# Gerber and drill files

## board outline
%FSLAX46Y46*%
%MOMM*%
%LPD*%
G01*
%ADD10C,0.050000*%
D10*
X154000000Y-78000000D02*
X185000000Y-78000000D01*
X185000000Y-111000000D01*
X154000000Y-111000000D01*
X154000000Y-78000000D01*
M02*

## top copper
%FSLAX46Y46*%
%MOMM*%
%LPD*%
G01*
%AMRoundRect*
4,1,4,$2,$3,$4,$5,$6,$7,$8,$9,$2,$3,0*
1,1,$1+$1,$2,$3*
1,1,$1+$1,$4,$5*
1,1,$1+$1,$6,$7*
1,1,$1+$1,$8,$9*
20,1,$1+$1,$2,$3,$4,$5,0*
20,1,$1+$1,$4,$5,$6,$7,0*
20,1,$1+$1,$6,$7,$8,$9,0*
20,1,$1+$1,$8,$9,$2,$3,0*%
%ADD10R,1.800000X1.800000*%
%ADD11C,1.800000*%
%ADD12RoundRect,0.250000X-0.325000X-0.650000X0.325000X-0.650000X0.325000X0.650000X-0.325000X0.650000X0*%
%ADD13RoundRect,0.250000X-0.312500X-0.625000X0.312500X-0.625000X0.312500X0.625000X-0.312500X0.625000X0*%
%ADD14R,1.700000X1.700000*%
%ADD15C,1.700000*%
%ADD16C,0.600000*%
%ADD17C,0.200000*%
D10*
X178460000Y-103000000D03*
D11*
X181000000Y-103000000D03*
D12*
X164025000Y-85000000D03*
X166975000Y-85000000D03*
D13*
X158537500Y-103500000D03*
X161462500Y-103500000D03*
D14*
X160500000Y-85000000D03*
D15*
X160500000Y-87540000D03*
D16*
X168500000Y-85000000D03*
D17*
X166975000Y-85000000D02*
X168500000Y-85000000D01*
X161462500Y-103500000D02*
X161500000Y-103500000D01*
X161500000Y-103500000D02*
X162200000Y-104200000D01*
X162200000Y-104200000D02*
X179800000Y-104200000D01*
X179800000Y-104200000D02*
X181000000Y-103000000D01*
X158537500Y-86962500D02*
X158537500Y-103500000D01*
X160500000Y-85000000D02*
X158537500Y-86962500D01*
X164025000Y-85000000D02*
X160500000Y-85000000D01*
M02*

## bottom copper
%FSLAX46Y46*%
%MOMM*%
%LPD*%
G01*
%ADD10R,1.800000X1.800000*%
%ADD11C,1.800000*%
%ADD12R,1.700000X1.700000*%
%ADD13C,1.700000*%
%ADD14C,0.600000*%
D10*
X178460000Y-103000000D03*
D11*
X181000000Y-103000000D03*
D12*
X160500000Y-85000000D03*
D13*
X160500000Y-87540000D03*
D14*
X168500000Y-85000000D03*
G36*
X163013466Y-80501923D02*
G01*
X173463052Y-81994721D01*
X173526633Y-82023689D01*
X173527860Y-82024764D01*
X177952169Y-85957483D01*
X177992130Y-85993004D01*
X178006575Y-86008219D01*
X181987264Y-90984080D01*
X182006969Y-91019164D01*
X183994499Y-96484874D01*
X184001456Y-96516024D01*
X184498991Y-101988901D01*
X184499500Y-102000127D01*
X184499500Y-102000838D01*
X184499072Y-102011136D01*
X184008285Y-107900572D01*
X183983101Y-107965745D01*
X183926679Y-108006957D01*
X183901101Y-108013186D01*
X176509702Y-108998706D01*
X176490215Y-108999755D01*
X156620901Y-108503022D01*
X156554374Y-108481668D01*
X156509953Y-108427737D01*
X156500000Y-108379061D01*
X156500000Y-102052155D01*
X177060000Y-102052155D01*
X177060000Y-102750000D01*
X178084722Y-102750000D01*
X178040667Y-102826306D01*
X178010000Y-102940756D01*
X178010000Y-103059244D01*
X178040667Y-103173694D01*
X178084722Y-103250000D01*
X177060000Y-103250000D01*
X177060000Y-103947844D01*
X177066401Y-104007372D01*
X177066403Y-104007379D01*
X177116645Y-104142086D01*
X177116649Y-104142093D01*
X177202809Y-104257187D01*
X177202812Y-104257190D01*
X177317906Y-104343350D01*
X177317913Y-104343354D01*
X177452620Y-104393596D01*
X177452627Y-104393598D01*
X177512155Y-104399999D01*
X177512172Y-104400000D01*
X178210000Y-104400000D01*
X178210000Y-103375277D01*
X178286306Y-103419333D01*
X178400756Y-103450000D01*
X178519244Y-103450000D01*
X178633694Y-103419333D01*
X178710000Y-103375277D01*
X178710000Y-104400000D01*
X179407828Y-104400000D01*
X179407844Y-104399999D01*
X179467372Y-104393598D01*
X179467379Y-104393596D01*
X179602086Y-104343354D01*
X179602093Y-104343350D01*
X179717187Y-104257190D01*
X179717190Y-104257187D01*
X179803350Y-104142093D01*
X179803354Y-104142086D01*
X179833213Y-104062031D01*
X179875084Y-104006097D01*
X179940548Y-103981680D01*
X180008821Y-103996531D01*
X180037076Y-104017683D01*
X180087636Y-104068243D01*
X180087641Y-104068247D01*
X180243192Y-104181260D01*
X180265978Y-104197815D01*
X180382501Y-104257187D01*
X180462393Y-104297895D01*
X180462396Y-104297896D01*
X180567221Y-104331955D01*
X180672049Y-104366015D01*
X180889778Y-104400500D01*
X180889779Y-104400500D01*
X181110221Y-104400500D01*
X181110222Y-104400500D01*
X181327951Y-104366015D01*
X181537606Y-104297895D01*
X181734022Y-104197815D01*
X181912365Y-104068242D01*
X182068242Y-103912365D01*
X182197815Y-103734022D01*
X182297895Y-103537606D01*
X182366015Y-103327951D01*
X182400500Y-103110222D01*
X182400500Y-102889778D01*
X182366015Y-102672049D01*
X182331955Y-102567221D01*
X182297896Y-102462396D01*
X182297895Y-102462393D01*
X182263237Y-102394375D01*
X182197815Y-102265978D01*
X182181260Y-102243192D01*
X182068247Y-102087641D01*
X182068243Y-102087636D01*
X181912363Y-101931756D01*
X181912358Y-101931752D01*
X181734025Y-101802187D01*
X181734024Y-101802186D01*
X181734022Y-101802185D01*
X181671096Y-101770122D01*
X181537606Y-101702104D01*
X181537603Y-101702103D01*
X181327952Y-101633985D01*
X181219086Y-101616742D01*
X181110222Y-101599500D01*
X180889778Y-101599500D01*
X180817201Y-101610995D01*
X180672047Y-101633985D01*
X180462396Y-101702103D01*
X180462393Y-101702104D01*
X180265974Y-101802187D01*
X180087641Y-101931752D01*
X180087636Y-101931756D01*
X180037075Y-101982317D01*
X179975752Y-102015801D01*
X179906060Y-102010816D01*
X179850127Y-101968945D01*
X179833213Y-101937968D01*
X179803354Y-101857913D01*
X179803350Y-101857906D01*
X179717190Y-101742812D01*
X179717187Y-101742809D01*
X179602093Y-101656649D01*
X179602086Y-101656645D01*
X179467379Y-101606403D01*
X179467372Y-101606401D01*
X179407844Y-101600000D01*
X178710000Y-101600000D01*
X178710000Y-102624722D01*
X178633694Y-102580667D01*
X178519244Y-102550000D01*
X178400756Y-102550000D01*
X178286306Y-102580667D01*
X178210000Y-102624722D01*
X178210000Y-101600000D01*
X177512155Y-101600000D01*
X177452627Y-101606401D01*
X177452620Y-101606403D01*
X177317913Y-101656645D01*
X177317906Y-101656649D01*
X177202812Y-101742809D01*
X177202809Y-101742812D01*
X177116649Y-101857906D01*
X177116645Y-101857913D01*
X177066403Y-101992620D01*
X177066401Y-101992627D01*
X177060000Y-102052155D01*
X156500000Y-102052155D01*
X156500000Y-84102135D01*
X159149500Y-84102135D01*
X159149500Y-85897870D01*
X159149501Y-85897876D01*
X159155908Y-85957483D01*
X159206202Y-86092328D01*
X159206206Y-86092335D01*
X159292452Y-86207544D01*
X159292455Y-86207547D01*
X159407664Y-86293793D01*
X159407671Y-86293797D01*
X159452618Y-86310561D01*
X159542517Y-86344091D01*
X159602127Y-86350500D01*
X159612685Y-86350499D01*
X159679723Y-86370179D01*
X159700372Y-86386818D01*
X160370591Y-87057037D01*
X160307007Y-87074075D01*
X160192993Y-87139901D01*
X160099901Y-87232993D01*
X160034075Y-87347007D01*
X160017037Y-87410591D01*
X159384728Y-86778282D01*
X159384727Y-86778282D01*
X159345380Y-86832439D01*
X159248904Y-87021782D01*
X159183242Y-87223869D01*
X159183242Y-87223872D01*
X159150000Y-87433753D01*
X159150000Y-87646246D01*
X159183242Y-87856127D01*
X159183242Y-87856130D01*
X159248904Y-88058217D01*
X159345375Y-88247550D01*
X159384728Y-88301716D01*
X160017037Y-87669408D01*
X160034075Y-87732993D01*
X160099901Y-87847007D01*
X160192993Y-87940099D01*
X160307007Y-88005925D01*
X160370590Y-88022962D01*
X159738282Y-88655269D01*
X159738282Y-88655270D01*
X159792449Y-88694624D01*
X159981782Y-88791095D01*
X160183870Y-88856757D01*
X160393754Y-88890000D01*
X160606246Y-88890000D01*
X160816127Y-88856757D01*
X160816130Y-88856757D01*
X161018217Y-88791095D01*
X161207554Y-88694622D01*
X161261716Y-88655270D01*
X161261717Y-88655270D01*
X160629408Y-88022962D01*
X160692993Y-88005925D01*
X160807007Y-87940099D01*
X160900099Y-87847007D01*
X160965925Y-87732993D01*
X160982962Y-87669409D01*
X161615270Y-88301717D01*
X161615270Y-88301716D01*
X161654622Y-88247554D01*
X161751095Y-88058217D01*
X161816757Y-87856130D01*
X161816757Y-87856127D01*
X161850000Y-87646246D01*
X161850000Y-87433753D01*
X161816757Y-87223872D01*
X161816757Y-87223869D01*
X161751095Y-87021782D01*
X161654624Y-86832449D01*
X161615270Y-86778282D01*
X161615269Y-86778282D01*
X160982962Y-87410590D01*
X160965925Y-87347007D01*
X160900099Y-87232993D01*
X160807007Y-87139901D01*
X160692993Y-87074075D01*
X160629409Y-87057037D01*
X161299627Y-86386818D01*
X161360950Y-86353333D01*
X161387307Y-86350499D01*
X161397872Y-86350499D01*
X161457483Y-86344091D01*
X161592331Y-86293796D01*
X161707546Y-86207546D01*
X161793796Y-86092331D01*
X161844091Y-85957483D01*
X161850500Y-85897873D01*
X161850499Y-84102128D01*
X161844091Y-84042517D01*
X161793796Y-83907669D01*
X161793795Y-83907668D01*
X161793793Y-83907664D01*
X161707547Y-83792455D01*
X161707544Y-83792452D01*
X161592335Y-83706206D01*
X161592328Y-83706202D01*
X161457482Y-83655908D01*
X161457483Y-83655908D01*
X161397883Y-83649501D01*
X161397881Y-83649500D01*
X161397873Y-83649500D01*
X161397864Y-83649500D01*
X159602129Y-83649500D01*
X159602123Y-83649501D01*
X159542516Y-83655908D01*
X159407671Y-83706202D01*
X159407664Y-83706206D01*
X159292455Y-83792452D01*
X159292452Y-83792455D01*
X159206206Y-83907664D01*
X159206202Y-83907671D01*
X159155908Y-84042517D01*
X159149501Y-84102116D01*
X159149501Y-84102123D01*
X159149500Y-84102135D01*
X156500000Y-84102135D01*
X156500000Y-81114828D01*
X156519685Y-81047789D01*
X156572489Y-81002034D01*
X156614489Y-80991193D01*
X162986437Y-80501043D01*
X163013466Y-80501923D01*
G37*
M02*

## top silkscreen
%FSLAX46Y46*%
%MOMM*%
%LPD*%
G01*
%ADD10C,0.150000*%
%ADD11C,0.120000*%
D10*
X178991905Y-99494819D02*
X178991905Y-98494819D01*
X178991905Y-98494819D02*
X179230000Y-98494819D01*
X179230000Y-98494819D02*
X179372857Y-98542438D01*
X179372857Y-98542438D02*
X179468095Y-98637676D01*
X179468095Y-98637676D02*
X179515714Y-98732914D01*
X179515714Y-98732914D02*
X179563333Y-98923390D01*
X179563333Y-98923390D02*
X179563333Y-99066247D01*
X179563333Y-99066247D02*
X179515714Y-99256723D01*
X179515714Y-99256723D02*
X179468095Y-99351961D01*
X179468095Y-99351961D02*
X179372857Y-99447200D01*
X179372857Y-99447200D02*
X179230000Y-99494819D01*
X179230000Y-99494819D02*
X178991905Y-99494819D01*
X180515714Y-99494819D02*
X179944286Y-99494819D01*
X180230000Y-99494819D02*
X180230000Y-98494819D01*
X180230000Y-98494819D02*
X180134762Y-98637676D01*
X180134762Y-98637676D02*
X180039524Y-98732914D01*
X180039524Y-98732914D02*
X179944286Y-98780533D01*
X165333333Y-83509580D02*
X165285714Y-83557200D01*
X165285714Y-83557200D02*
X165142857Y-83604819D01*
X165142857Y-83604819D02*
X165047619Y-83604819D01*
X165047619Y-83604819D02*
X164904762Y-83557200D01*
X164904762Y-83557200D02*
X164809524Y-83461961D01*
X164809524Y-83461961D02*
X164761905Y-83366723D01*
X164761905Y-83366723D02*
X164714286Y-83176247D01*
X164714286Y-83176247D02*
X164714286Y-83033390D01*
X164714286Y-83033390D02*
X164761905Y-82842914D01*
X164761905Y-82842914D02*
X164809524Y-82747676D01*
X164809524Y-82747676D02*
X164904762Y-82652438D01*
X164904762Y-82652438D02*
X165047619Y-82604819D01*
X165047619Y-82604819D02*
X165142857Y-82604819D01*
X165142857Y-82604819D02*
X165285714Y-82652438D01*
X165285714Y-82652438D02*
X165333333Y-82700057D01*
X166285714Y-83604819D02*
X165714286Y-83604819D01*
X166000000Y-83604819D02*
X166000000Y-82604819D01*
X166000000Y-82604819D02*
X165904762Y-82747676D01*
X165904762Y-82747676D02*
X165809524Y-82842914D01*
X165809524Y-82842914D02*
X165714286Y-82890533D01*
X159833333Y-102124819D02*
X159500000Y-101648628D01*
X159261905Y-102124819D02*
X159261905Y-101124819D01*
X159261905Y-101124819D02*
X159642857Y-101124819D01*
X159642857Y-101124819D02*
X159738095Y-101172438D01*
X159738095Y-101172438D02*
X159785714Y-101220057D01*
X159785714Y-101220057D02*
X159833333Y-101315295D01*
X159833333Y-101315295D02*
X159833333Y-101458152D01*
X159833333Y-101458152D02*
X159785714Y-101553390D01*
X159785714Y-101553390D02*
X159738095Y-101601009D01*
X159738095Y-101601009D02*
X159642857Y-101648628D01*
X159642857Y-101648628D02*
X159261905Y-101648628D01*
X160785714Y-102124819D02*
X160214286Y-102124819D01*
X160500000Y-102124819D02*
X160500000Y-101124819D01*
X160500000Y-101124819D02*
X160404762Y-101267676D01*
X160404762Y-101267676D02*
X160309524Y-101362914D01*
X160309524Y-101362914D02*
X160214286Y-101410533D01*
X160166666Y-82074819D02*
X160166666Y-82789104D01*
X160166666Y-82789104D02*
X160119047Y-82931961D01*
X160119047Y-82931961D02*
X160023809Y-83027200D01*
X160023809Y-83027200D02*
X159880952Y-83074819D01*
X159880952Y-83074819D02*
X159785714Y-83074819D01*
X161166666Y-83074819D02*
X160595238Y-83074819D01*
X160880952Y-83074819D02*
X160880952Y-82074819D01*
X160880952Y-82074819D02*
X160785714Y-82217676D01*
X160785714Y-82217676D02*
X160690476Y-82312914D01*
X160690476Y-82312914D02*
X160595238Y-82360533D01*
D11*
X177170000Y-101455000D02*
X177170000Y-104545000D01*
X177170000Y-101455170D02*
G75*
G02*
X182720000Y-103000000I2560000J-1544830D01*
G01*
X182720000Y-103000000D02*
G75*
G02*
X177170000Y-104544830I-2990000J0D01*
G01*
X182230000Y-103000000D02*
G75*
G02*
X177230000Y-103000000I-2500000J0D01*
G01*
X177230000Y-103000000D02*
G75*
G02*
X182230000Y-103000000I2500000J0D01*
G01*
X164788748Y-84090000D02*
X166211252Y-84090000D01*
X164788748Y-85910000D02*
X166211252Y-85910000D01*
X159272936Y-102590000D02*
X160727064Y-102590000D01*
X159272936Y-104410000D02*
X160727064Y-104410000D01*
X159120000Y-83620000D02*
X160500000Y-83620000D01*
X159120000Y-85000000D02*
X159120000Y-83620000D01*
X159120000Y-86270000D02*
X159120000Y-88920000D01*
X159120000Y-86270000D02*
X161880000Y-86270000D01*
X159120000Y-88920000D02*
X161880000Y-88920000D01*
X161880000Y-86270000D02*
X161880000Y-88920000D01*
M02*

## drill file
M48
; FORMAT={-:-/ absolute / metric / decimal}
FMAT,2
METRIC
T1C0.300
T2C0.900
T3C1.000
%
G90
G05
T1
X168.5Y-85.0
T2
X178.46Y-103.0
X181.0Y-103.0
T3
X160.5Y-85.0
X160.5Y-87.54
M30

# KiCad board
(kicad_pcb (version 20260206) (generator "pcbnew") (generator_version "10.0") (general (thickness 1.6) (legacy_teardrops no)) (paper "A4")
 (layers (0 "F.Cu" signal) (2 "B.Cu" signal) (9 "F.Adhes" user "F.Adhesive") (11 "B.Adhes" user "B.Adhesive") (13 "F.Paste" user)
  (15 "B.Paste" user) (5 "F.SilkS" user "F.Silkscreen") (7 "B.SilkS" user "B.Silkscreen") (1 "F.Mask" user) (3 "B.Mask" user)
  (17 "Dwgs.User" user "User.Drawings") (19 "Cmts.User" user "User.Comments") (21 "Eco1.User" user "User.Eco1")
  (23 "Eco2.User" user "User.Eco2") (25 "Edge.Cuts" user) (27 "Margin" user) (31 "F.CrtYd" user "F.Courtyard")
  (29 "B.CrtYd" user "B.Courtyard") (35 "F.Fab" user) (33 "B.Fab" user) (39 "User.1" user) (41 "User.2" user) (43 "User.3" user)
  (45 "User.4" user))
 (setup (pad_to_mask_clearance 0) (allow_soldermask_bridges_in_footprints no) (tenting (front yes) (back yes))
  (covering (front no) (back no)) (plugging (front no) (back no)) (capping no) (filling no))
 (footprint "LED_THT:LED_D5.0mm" (layer "F.Cu") (at 178.46 103)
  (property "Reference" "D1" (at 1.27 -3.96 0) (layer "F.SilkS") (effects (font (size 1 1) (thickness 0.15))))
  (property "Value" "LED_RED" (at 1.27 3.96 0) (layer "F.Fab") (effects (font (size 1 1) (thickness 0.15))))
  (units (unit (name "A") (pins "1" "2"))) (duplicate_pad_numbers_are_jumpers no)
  (fp_line (start -1.29 -1.545) (end -1.29 1.545) (stroke (width 0.12) (type solid)) (layer "F.SilkS"))
  (fp_arc (start -1.29 -1.54483) (mid 2.071779 -2.880495) (end 4.26 0) (stroke (width 0.12) (type solid)) (layer "F.SilkS"))
  (fp_arc (start 4.26 0) (mid 2.071779 2.880495) (end -1.29 1.54483) (stroke (width 0.12) (type solid)) (layer "F.SilkS"))
  (fp_circle (center 1.27 0) (end 3.77 0) (stroke (width 0.12) (type solid)) (fill no) (layer "F.SilkS"))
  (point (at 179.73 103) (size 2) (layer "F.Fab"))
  (pad "1" thru_hole rect (at 0 0) (size 1.8 1.8) (drill 0.9) (layers "*.Cu" "*.Mask") (remove_unused_layers no) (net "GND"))
  (pad "2" thru_hole circle (at 2.54 0) (size 1.8 1.8) (drill 0.9) (layers "*.Cu" "*.Mask") (remove_unused_layers no) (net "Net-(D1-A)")))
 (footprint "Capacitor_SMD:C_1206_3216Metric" (layer "F.Cu") (at 165.5 85)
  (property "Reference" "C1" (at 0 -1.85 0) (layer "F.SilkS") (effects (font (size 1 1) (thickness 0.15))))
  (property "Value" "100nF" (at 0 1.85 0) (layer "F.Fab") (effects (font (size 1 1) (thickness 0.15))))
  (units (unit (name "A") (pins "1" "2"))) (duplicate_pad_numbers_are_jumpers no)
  (fp_line (start -0.711252 -0.91) (end 0.711252 -0.91) (stroke (width 0.12) (type solid)) (layer "F.SilkS"))
  (fp_line (start -0.711252 0.91) (end 0.711252 0.91) (stroke (width 0.12) (type solid)) (layer "F.SilkS"))
  (pad "1" smd roundrect (at -1.475 0) (size 1.15 1.8) (layers "F.Cu" "F.Mask" "F.Paste") (roundrect_rratio 0.217391) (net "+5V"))
  (pad "2" smd roundrect (at 1.475 0) (size 1.15 1.8) (layers "F.Cu" "F.Mask" "F.Paste") (roundrect_rratio 0.217391) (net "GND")))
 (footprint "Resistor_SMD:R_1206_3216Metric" (layer "F.Cu") (at 160 103.5)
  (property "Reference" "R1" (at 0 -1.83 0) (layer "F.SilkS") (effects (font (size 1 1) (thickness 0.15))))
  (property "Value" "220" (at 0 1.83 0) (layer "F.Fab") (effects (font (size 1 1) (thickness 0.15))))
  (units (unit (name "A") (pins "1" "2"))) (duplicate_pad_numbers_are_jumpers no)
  (fp_line (start -0.727064 -0.91) (end 0.727064 -0.91) (stroke (width 0.12) (type solid)) (layer "F.SilkS"))
  (fp_line (start -0.727064 0.91) (end 0.727064 0.91) (stroke (width 0.12) (type solid)) (layer "F.SilkS"))
  (pad "1" smd roundrect (at -1.4625 0) (size 1.125 1.75) (layers "F.Cu" "F.Mask" "F.Paste") (roundrect_rratio 0.222222) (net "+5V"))
  (pad "2" smd roundrect (at 1.4625 0) (size 1.125 1.75) (layers "F.Cu" "F.Mask" "F.Paste") (roundrect_rratio 0.222222) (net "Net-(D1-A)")))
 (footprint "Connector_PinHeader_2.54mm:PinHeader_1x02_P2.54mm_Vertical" (layer "F.Cu") (at 160.5 85)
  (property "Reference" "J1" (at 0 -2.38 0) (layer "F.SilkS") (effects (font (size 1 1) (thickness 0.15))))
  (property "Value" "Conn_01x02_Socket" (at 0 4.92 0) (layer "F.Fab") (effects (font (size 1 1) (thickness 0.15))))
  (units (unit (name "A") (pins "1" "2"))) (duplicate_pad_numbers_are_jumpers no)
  (fp_line (start -1.38 -1.38) (end 0 -1.38) (stroke (width 0.12) (type solid)) (layer "F.SilkS"))
  (fp_line (start -1.38 0) (end -1.38 -1.38) (stroke (width 0.12) (type solid)) (layer "F.SilkS"))
  (fp_line (start -1.38 1.27) (end -1.38 3.92) (stroke (width 0.12) (type solid)) (layer "F.SilkS"))
  (fp_line (start -1.38 1.27) (end 1.38 1.27) (stroke (width 0.12) (type solid)) (layer "F.SilkS"))
  (fp_line (start -1.38 3.92) (end 1.38 3.92) (stroke (width 0.12) (type solid)) (layer "F.SilkS"))
  (fp_line (start 1.38 1.27) (end 1.38 3.92) (stroke (width 0.12) (type solid)) (layer "F.SilkS"))
  (pad "1" thru_hole rect (at 0 0) (size 1.7 1.7) (drill 1) (layers "*.Cu" "*.Mask") (remove_unused_layers no) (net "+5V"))
  (pad "2" thru_hole circle (at 0 2.54) (size 1.7 1.7) (drill 1) (layers "*.Cu" "*.Mask") (remove_unused_layers no) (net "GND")))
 (gr_rect (start 154 78) (end 185 111) (stroke (width 0.05) (type default)) (fill no) (layer "Edge.Cuts"))
 (segment (start 166.975 85) (end 168.5 85) (width 0.2) (layer "F.Cu") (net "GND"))
 (via (at 168.5 85) (size 0.6) (drill 0.3) (layers "F.Cu" "B.Cu") (free yes) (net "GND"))
 (segment (start 161.4625 103.5) (end 161.5 103.5) (width 0.2) (layer "F.Cu") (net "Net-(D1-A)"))
 (segment (start 161.5 103.5) (end 162.2 104.2) (width 0.2) (layer "F.Cu") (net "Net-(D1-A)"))
 (segment (start 162.2 104.2) (end 179.8 104.2) (width 0.2) (layer "F.Cu") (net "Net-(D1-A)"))
 (segment (start 179.8 104.2) (end 181 103) (width 0.2) (layer "F.Cu") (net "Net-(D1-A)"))
 (segment (start 158.5375 86.9625) (end 158.5375 103.5) (width 0.2) (layer "F.Cu") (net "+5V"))
 (segment (start 160.5 85) (end 158.5375 86.9625) (width 0.2) (layer "F.Cu") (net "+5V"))
 (segment (start 164.025 85) (end 160.5 85) (width 0.2) (layer "F.Cu") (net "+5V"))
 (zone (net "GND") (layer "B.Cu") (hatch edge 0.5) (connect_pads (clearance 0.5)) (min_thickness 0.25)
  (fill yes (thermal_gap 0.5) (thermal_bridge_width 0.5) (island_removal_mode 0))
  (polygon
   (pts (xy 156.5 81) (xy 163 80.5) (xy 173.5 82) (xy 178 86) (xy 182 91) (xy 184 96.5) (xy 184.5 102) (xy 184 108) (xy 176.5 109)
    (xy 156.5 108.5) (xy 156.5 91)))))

